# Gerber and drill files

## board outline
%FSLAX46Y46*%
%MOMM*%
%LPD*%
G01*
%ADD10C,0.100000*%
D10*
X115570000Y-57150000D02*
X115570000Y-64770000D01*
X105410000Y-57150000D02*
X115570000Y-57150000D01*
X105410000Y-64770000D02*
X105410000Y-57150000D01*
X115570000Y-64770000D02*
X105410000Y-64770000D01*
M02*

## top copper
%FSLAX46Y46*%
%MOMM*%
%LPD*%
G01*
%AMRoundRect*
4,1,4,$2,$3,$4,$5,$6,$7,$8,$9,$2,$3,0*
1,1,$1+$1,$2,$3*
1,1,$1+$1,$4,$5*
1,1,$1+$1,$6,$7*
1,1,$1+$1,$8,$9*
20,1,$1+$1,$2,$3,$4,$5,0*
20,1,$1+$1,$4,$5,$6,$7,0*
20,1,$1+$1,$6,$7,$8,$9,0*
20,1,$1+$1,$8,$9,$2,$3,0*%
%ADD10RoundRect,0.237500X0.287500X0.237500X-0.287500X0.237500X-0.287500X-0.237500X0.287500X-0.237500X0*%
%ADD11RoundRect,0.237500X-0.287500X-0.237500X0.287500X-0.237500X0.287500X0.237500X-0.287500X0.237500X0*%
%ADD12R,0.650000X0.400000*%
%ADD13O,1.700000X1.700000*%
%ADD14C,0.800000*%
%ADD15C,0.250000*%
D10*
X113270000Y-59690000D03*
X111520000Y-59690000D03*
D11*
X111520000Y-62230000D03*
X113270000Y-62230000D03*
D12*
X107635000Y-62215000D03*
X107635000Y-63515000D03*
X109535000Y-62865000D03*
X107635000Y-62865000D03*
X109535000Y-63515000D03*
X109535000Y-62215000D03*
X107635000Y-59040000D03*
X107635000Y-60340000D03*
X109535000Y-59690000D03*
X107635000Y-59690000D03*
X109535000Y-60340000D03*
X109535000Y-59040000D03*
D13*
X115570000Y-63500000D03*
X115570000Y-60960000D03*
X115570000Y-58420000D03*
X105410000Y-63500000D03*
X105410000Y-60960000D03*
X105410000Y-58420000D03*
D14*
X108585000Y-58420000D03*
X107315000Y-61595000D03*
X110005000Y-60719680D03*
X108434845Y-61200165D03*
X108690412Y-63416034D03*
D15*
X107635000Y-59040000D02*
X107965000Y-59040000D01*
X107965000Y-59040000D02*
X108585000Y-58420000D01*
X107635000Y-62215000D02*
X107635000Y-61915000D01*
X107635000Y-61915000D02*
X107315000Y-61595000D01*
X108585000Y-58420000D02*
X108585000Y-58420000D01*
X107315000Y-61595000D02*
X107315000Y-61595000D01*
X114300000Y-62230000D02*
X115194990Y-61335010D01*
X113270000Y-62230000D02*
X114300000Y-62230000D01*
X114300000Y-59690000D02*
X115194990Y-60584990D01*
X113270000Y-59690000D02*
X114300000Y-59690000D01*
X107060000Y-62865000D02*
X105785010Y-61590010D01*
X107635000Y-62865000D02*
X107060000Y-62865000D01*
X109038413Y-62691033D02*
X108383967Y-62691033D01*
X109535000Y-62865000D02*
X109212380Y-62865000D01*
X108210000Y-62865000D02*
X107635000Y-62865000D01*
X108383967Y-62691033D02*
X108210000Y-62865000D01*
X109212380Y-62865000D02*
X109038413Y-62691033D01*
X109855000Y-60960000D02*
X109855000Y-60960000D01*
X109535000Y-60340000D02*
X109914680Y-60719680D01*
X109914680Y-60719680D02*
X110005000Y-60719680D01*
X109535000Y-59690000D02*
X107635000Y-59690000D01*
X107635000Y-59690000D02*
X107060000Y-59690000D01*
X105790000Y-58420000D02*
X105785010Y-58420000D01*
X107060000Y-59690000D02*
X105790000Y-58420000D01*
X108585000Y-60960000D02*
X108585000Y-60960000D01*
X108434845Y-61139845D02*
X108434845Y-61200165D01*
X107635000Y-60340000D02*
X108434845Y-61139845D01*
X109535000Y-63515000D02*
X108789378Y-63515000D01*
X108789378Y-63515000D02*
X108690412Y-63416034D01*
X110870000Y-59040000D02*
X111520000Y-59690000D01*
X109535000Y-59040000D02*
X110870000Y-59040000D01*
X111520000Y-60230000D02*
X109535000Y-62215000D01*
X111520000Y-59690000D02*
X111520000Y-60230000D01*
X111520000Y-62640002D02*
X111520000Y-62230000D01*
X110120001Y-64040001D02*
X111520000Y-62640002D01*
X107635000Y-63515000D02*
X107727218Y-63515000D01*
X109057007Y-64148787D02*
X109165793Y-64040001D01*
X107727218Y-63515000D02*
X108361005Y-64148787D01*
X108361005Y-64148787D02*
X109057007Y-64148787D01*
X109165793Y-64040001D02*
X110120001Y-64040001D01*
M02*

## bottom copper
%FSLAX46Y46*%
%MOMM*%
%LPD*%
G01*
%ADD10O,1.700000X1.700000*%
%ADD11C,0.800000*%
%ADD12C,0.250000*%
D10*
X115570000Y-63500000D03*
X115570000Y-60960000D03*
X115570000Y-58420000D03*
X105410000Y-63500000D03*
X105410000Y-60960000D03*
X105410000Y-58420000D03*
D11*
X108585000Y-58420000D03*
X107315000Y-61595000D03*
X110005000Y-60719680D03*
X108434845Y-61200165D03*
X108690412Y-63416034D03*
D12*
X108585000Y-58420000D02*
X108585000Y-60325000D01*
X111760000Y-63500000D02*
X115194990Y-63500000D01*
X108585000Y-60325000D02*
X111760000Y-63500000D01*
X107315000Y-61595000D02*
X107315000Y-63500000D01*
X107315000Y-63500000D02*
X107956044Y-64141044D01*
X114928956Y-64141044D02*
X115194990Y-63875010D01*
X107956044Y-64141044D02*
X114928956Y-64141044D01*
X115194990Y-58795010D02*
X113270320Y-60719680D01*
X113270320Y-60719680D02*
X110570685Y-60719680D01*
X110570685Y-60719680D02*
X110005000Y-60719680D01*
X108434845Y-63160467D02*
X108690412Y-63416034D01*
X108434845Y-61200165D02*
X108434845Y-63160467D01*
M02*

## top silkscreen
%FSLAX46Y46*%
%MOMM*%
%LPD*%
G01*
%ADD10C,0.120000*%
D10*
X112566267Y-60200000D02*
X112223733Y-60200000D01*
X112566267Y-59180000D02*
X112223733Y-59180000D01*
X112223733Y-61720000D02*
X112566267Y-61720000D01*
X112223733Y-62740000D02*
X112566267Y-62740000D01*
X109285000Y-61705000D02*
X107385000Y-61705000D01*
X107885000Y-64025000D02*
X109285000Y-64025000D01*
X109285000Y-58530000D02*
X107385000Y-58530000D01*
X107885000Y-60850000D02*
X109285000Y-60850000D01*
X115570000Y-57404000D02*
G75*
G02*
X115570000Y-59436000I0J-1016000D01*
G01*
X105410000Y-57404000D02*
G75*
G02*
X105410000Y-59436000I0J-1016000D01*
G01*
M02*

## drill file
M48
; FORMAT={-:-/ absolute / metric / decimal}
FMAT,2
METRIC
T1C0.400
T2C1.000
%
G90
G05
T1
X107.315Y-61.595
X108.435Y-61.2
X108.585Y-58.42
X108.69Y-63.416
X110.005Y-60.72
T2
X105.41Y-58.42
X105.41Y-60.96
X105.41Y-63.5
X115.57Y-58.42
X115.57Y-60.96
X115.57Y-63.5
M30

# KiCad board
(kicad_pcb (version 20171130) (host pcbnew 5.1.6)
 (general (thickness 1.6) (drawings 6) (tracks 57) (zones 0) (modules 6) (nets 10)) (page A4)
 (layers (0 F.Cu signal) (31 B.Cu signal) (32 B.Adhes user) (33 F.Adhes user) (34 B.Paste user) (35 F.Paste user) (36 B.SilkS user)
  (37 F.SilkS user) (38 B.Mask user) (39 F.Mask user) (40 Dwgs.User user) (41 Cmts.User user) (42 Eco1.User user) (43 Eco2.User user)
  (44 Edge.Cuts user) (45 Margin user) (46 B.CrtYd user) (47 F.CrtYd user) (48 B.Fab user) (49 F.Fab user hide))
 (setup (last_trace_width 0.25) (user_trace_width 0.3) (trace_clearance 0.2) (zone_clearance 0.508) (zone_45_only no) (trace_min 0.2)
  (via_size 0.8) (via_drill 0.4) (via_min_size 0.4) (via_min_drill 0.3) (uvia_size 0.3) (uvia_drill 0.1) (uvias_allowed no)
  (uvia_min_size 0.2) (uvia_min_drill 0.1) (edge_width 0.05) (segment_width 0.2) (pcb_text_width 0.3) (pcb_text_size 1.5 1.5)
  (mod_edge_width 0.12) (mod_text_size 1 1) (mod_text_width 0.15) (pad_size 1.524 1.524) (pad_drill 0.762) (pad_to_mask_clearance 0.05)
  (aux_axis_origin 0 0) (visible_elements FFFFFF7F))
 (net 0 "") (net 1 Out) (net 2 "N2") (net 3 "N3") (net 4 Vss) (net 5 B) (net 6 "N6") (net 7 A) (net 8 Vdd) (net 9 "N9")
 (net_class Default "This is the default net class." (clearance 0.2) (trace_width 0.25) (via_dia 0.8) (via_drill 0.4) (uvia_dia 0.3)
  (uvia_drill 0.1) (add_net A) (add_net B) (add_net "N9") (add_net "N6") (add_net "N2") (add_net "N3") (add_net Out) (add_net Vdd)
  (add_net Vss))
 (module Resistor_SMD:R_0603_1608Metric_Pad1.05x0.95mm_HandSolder (layer F.Cu) (at 112.395 59.69 180)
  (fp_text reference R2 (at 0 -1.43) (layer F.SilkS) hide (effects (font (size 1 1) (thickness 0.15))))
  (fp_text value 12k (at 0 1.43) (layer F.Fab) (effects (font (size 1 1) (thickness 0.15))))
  (fp_line (start -0.171267 -0.51) (end 0.171267 -0.51) (layer F.SilkS) (width 0.12))
  (fp_line (start -0.171267 0.51) (end 0.171267 0.51) (layer F.SilkS) (width 0.12))
  (pad 1 smd roundrect (at -0.875 0 180) (size 1.05 0.95) (layers F.Cu F.Paste F.Mask) (roundrect_rratio 0.25) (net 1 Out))
  (pad 2 smd roundrect (at 0.875 0 180) (size 1.05 0.95) (layers F.Cu F.Paste F.Mask) (roundrect_rratio 0.25) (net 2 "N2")))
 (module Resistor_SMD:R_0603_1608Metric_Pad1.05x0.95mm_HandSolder (layer F.Cu) (at 112.395 62.23)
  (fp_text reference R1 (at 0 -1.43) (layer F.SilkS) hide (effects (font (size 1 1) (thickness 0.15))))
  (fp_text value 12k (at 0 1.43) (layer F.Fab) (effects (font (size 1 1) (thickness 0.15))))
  (fp_line (start -0.171267 -0.51) (end 0.171267 -0.51) (layer F.SilkS) (width 0.12))
  (fp_line (start -0.171267 0.51) (end 0.171267 0.51) (layer F.SilkS) (width 0.12))
  (pad 1 smd roundrect (at -0.875 0) (size 1.05 0.95) (layers F.Cu F.Paste F.Mask) (roundrect_rratio 0.25) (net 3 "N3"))
  (pad 2 smd roundrect (at 0.875 0) (size 1.05 0.95) (layers F.Cu F.Paste F.Mask) (roundrect_rratio 0.25) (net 1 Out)))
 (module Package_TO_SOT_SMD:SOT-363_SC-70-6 (layer F.Cu) (at 108.585 62.865)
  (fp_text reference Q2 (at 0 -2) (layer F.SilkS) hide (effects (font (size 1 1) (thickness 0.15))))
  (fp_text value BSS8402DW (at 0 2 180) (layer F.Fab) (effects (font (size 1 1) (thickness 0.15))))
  (fp_line (start 0.7 -1.16) (end -1.2 -1.16) (layer F.SilkS) (width 0.12))
  (fp_line (start -0.7 1.16) (end 0.7 1.16) (layer F.SilkS) (width 0.12))
  (pad 1 smd rect (at -0.95 -0.65) (size 0.65 0.4) (layers F.Cu F.Paste F.Mask) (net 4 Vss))
  (pad 3 smd rect (at -0.95 0.65) (size 0.65 0.4) (layers F.Cu F.Paste F.Mask) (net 3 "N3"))
  (pad 5 smd rect (at 0.95 0) (size 0.65 0.4) (layers F.Cu F.Paste F.Mask) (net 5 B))
  (pad 2 smd rect (at -0.95 0) (size 0.65 0.4) (layers F.Cu F.Paste F.Mask) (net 5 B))
  (pad 4 smd rect (at 0.95 0.65) (size 0.65 0.4) (layers F.Cu F.Paste F.Mask) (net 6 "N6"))
  (pad 6 smd rect (at 0.95 -0.65) (size 0.65 0.4) (layers F.Cu F.Paste F.Mask) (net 2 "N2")))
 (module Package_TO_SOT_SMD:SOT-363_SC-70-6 (layer F.Cu) (at 108.585 59.69)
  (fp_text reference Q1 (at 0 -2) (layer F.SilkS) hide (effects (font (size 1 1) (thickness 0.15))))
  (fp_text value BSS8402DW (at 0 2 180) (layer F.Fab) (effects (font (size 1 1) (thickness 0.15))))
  (fp_line (start 0.7 -1.16) (end -1.2 -1.16) (layer F.SilkS) (width 0.12))
  (fp_line (start -0.7 1.16) (end 0.7 1.16) (layer F.SilkS) (width 0.12))
  (pad 1 smd rect (at -0.95 -0.65) (size 0.65 0.4) (layers F.Cu F.Paste F.Mask) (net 4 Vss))
  (pad 3 smd rect (at -0.95 0.65) (size 0.65 0.4) (layers F.Cu F.Paste F.Mask) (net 6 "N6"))
  (pad 5 smd rect (at 0.95 0) (size 0.65 0.4) (layers F.Cu F.Paste F.Mask) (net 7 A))
  (pad 2 smd rect (at -0.95 0) (size 0.65 0.4) (layers F.Cu F.Paste F.Mask) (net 7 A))
  (pad 4 smd rect (at 0.95 0.65) (size 0.65 0.4) (layers F.Cu F.Paste F.Mask) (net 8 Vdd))
  (pad 6 smd rect (at 0.95 -0.65) (size 0.65 0.4) (layers F.Cu F.Paste F.Mask) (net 2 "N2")))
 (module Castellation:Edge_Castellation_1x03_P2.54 (layer F.Cu) (at 115.57 58.42)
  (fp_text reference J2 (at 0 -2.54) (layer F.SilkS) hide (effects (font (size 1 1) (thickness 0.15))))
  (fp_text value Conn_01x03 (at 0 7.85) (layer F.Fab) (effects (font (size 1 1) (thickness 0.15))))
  (fp_arc (start 0 0) (end 0 1.016) (angle -180) (layer F.SilkS) (width 0.12))
  (pad 3 thru_hole oval (at 0 5.08) (size 1.7 1.7) (drill 1) (layers *.Cu *.Mask) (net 4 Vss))
  (pad 2 thru_hole oval (at 0 2.54) (size 1.7 1.7) (drill 1) (layers *.Cu *.Mask) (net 1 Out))
  (pad 1 thru_hole oval (at 0 0) (size 1.7 1.7) (drill 1) (layers *.Cu *.Mask) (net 8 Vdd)))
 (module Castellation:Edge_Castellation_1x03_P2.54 (layer F.Cu) (at 105.41 58.42)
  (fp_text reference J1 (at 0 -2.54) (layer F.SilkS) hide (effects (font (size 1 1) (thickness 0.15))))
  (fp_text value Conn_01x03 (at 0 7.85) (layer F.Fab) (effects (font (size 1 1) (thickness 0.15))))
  (fp_arc (start 0 0) (end 0 1.016) (angle -180) (layer F.SilkS) (width 0.12))
  (pad 3 thru_hole oval (at 0 5.08) (size 1.7 1.7) (drill 1) (layers *.Cu *.Mask) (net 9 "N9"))
  (pad 2 thru_hole oval (at 0 2.54) (size 1.7 1.7) (drill 1) (layers *.Cu *.Mask) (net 5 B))
  (pad 1 thru_hole oval (at 0 0) (size 1.7 1.7) (drill 1) (layers *.Cu *.Mask) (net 7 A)))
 (gr_line (start 115.57 57.15) (end 115.57 64.77) (layer Edge.Cuts) (width 0.1))
 (gr_line (start 105.41 57.15) (end 115.57 57.15) (layer Edge.Cuts) (width 0.1))
 (gr_line (start 105.41 64.77) (end 105.41 57.15) (layer Edge.Cuts) (width 0.1))
 (gr_line (start 115.57 64.77) (end 105.41 64.77) (layer Edge.Cuts) (width 0.1))
 (segment (start 107.635 59.04) (end 107.965 59.04) (width 0.25) (layer F.Cu) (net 4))
 (segment (start 107.965 59.04) (end 108.585 58.42) (width 0.25) (layer F.Cu) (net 4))
 (segment (start 107.635 62.215) (end 107.635 61.915) (width 0.25) (layer F.Cu) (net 4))
 (segment (start 107.635 61.915) (end 107.315 61.595) (width 0.25) (layer F.Cu) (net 4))
 (segment (start 108.585 58.42) (end 108.585 58.42) (width 0.25) (layer F.Cu) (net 4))
 (via (at 108.585 58.42) (size 0.8) (drill 0.4) (layers F.Cu B.Cu) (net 4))
 (segment (start 107.315 61.595) (end 107.315 61.595) (width 0.25) (layer F.Cu) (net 4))
 (via (at 107.315 61.595) (size 0.8) (drill 0.4) (layers F.Cu B.Cu) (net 4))
 (segment (start 108.585 58.42) (end 108.585 60.325) (width 0.25) (layer B.Cu) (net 4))
 (segment (start 111.76 63.5) (end 115.19499 63.5) (width 0.25) (layer B.Cu) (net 4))
 (segment (start 108.585 60.325) (end 111.76 63.5) (width 0.25) (layer B.Cu) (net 4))
 (segment (start 107.315 61.595) (end 107.315 63.5) (width 0.25) (layer B.Cu) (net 4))
 (segment (start 107.315 63.5) (end 107.956044 64.141044) (width 0.25) (layer B.Cu) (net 4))
 (segment (start 114.928956 64.141044) (end 115.19499 63.87501) (width 0.25) (layer B.Cu) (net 4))
 (segment (start 107.956044 64.141044) (end 114.928956 64.141044) (width 0.25) (layer B.Cu) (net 4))
 (segment (start 114.3 62.23) (end 115.19499 61.33501) (width 0.25) (layer F.Cu) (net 1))
 (segment (start 113.27 62.23) (end 114.3 62.23) (width 0.25) (layer F.Cu) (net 1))
 (segment (start 114.3 59.69) (end 115.19499 60.58499) (width 0.25) (layer F.Cu) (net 1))
 (segment (start 113.27 59.69) (end 114.3 59.69) (width 0.25) (layer F.Cu) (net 1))
 (segment (start 107.06 62.865) (end 105.78501 61.59001) (width 0.25) (layer F.Cu) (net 5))
 (segment (start 107.635 62.865) (end 107.06 62.865) (width 0.25) (layer F.Cu) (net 5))
 (segment (start 109.038413 62.691033) (end 108.383967 62.691033) (width 0.25) (layer F.Cu) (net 5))
 (segment (start 109.535 62.865) (end 109.21238 62.865) (width 0.25) (layer F.Cu) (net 5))
 (segment (start 108.21 62.865) (end 107.635 62.865) (width 0.25) (layer F.Cu) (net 5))
 (segment (start 108.383967 62.691033) (end 108.21 62.865) (width 0.25) (layer F.Cu) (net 5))
 (segment (start 109.21238 62.865) (end 109.038413 62.691033) (width 0.25) (layer F.Cu) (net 5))
 (segment (start 109.855 60.96) (end 109.855 60.96) (width 0.25) (layer F.Cu) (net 8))
 (via (at 110.005 60.71968) (size 0.8) (drill 0.4) (layers F.Cu B.Cu) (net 8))
 (segment (start 109.535 60.34) (end 109.91468 60.71968) (width 0.25) (layer F.Cu) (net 8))
 (segment (start 115.19499 58.79501) (end 113.27032 60.71968) (width 0.25) (layer B.Cu) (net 8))
 (segment (start 113.27032 60.71968) (end 110.570685 60.71968) (width 0.25) (layer B.Cu) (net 8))
 (segment (start 110.570685 60.71968) (end 110.005 60.71968) (width 0.25) (layer B.Cu) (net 8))
 (segment (start 109.91468 60.71968) (end 110.005 60.71968) (width 0.25) (layer F.Cu) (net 8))
 (segment (start 109.535 59.69) (end 107.635 59.69) (width 0.25) (layer F.Cu) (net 7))
 (segment (start 107.635 59.69) (end 107.06 59.69) (width 0.25) (layer F.Cu) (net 7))
 (segment (start 105.79 58.42) (end 105.78501 58.42) (width 0.25) (layer F.Cu) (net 7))
 (segment (start 107.06 59.69) (end 105.79 58.42) (width 0.25) (layer F.Cu) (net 7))
 (segment (start 108.585 60.96) (end 108.585 60.96) (width 0.25) (layer F.Cu) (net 6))
 (via (at 108.434845 61.200165) (size 0.8) (drill 0.4) (layers F.Cu B.Cu) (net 6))
 (segment (start 108.434845 61.139845) (end 108.434845 61.200165) (width 0.25) (layer F.Cu) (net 6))
 (segment (start 107.635 60.34) (end 108.434845 61.139845) (width 0.25) (layer F.Cu) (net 6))
 (segment (start 108.434845 63.160467) (end 108.690412 63.416034) (width 0.25) (layer B.Cu) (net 6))
 (segment (start 108.434845 61.200165) (end 108.434845 63.160467) (width 0.25) (layer B.Cu) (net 6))
 (segment (start 109.535 63.515) (end 108.789378 63.515) (width 0.25) (layer F.Cu) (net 6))
 (segment (start 108.789378 63.515) (end 108.690412 63.416034) (width 0.25) (layer F.Cu) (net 6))
 (via (at 108.690412 63.416034) (size 0.8) (drill 0.4) (layers F.Cu B.Cu) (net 6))
 (segment (start 110.87 59.04) (end 111.52 59.69) (width 0.25) (layer F.Cu) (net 2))
 (segment (start 109.535 59.04) (end 110.87 59.04) (width 0.25) (layer F.Cu) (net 2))
 (segment (start 111.52 60.23) (end 109.535 62.215) (width 0.25) (layer F.Cu) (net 2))
 (segment (start 111.52 59.69) (end 111.52 60.23) (width 0.25) (layer F.Cu) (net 2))
 (segment (start 111.52 62.640002) (end 111.52 62.23) (width 0.25) (layer F.Cu) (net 3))
 (segment (start 110.120001 64.040001) (end 111.52 62.640002) (width 0.25) (layer F.Cu) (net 3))
 (segment (start 107.635 63.515) (end 107.727218 63.515) (width 0.25) (layer F.Cu) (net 3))
 (segment (start 109.057007 64.148787) (end 109.165793 64.040001) (width 0.25) (layer F.Cu) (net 3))
 (segment (start 107.727218 63.515) (end 108.361005 64.148787) (width 0.25) (layer F.Cu) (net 3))
 (segment (start 108.361005 64.148787) (end 109.057007 64.148787) (width 0.25) (layer F.Cu) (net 3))
 (segment (start 109.165793 64.040001) (end 110.120001 64.040001) (width 0.25) (layer F.Cu) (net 3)))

